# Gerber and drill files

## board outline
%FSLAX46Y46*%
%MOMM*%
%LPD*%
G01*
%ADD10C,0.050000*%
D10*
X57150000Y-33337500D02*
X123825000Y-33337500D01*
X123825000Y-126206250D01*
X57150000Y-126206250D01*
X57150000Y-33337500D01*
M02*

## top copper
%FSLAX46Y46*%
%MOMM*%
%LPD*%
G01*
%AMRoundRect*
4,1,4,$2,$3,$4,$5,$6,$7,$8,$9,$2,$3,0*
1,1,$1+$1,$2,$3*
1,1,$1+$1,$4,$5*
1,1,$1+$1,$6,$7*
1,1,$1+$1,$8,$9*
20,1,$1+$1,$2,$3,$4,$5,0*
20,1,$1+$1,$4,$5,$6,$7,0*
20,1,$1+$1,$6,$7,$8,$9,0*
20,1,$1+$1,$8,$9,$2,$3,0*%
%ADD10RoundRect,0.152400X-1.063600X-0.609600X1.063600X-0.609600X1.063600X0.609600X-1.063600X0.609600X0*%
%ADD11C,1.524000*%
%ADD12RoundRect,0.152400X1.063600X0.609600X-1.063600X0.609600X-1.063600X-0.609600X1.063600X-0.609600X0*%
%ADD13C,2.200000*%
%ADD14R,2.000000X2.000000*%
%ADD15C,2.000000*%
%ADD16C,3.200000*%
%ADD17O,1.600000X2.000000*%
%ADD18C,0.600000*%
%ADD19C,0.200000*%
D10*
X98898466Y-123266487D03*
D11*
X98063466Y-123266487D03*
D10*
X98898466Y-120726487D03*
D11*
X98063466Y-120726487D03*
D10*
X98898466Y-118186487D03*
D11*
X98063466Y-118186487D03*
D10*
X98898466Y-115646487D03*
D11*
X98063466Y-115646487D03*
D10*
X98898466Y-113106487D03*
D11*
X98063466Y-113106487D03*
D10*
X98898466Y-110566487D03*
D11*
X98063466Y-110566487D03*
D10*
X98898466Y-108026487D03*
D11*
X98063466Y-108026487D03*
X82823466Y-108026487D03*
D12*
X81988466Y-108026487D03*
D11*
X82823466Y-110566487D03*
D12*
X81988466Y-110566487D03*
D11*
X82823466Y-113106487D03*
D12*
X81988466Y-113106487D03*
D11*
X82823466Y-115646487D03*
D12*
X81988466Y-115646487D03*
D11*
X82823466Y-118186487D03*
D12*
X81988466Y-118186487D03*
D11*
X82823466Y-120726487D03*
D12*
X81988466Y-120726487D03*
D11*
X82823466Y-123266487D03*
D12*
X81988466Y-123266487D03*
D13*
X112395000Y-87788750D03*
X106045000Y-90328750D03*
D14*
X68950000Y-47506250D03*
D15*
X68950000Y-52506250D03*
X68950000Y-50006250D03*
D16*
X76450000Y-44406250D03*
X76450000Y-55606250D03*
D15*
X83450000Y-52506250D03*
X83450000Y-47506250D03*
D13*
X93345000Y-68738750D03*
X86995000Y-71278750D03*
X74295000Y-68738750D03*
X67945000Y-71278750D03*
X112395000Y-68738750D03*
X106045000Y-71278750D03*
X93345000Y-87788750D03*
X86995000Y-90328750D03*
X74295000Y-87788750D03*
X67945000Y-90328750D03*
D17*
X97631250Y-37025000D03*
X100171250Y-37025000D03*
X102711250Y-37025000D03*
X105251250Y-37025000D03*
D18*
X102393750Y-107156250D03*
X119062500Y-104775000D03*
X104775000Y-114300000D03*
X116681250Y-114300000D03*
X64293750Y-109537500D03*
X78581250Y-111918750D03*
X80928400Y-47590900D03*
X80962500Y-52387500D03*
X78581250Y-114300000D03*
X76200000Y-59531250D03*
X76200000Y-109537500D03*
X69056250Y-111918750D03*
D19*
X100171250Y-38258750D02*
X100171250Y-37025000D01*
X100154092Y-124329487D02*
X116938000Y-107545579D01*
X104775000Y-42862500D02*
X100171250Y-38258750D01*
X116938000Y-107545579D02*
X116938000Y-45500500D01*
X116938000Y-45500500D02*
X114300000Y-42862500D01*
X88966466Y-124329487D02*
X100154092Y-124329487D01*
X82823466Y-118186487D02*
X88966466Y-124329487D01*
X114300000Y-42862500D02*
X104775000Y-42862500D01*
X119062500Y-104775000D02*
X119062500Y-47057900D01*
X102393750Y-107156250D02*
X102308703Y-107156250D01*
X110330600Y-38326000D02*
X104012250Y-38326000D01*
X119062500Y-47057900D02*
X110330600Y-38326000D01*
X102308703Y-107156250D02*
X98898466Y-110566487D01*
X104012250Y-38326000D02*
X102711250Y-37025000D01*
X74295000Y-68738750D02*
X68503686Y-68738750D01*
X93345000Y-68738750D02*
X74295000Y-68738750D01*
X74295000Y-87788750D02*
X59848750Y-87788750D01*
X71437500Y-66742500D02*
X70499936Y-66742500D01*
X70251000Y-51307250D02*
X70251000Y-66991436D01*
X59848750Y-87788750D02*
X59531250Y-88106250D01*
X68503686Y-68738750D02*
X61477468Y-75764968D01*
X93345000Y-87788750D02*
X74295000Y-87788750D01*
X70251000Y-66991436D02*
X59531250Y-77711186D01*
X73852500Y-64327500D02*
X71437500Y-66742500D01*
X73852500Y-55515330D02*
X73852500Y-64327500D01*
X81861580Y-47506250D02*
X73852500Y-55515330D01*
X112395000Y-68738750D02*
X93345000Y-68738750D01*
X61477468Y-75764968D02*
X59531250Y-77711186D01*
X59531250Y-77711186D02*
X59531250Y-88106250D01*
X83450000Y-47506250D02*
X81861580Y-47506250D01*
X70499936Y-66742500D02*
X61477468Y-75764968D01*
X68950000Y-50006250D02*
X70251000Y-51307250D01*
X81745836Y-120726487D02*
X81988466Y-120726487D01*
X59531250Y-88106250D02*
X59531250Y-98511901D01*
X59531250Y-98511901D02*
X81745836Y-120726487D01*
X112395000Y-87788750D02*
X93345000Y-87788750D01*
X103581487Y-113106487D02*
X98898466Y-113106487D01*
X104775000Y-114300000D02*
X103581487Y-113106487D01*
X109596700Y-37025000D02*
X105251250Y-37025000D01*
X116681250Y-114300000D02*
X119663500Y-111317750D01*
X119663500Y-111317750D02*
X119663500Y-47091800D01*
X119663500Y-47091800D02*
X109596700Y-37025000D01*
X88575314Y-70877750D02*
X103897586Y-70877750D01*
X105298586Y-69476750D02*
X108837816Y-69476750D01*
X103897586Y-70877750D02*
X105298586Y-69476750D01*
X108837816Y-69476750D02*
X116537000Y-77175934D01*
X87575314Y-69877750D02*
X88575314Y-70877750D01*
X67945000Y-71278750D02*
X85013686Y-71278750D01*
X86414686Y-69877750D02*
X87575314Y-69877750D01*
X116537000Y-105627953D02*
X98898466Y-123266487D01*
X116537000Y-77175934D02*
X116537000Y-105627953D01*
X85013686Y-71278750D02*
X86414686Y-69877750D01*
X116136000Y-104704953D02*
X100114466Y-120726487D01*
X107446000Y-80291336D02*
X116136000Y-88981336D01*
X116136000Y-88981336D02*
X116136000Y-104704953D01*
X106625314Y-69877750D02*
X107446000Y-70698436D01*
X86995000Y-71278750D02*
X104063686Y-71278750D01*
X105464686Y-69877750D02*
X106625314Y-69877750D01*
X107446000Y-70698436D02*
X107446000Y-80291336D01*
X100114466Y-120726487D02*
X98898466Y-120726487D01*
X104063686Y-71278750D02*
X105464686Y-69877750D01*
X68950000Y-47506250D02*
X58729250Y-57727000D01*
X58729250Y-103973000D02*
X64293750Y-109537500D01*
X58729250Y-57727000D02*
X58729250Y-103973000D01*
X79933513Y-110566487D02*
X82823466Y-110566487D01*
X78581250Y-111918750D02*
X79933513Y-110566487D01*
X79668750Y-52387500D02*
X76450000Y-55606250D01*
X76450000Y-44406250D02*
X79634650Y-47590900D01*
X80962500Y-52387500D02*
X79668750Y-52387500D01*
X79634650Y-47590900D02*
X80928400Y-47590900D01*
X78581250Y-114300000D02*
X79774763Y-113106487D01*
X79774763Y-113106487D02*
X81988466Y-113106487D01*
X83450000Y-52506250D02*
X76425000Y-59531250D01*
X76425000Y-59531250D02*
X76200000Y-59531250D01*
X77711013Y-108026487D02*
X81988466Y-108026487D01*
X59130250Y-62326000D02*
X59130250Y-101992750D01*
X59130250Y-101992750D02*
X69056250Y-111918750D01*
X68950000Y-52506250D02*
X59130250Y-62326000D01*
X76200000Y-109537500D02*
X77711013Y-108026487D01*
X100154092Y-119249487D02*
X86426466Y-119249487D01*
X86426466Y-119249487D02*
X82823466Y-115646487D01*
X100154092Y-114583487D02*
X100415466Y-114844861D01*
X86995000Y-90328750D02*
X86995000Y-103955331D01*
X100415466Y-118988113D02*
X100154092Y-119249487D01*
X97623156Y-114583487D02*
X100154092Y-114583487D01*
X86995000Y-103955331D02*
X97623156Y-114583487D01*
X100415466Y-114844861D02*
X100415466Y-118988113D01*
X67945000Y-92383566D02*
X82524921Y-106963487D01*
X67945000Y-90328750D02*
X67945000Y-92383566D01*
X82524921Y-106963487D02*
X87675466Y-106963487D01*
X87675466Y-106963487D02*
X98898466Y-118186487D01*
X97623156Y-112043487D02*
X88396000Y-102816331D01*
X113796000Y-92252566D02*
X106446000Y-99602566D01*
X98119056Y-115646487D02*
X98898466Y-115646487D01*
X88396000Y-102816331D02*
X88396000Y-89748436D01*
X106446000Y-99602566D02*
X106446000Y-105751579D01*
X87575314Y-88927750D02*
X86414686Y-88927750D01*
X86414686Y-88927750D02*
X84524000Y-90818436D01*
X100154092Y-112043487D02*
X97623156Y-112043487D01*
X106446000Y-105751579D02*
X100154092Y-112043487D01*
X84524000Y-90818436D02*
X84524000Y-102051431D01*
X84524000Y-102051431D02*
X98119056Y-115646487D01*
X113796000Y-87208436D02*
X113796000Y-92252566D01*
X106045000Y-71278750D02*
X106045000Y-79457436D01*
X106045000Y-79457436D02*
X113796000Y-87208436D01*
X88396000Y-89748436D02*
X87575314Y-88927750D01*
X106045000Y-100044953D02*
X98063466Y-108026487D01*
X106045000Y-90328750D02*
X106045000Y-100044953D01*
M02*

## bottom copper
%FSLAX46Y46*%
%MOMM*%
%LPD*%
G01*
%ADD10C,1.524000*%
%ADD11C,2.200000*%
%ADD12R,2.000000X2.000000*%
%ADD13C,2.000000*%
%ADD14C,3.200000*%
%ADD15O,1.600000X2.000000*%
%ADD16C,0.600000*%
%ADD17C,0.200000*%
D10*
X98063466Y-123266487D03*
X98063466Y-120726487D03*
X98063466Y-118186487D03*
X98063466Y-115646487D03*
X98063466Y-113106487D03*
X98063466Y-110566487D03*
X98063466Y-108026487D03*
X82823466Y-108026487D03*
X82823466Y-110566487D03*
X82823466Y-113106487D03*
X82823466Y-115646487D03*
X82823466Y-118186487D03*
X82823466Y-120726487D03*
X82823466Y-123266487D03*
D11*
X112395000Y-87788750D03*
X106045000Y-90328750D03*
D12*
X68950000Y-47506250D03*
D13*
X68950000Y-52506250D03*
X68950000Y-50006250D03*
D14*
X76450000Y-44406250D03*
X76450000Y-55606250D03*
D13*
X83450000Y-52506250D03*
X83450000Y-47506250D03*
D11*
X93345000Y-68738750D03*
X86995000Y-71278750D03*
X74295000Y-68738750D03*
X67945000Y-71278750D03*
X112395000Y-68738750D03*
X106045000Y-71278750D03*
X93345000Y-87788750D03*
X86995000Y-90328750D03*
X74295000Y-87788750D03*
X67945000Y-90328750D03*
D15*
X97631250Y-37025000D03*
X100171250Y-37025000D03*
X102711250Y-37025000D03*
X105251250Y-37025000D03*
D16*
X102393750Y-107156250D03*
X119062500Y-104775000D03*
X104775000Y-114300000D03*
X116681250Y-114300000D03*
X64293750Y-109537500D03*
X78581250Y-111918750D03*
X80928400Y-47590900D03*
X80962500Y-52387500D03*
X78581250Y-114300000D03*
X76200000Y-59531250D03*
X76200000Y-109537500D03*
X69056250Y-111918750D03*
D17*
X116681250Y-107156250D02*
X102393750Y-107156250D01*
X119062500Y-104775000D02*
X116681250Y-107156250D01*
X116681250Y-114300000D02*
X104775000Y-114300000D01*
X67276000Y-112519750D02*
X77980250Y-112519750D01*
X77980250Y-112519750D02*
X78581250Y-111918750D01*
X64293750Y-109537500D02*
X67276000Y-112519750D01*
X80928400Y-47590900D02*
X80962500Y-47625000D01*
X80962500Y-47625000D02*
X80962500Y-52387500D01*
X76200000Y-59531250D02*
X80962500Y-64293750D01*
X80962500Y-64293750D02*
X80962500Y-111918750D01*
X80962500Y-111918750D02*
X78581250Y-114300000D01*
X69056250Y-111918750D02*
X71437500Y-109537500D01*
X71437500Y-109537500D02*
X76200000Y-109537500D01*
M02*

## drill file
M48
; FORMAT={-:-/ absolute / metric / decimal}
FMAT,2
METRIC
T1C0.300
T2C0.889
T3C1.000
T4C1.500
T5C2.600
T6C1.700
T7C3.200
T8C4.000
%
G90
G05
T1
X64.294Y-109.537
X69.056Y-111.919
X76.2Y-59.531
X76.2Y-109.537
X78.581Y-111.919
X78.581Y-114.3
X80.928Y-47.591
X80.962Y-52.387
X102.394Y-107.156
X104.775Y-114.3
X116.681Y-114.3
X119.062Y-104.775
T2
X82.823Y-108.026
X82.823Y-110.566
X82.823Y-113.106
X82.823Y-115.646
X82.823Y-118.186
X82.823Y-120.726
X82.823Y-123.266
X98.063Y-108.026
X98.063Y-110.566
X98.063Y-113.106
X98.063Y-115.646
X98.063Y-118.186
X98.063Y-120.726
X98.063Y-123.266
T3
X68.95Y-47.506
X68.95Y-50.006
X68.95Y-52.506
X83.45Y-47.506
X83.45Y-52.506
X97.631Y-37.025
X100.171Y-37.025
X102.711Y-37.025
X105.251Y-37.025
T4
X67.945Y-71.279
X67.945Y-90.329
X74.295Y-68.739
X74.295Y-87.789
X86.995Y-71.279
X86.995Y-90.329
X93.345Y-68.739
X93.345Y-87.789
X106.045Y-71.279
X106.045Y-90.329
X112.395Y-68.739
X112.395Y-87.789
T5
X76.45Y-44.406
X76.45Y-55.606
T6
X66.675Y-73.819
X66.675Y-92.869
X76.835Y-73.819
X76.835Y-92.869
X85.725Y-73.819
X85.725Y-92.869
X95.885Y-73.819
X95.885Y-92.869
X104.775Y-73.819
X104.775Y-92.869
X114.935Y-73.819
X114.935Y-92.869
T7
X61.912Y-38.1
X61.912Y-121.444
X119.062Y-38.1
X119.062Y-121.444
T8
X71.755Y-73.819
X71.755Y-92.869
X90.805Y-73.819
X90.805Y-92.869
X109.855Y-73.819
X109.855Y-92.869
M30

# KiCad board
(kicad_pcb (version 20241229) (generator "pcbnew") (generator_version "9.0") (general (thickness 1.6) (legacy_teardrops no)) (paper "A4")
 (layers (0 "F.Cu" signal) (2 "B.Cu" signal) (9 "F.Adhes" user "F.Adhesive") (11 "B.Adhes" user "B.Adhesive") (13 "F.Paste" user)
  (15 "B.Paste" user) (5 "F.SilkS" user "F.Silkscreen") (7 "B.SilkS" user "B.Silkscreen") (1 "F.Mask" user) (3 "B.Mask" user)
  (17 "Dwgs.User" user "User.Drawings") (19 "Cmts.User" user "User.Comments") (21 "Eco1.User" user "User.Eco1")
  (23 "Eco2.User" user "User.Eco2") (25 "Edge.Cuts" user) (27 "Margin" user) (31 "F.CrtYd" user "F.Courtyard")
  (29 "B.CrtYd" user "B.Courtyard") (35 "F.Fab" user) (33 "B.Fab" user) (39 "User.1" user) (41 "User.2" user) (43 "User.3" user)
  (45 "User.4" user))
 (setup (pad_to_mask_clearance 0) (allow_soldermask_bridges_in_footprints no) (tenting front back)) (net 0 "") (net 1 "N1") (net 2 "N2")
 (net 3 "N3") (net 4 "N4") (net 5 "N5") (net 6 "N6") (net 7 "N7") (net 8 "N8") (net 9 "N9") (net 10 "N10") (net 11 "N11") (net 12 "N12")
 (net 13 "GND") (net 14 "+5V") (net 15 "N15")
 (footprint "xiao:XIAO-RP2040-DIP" (layer "F.Cu") (at 90.443466 115.646487 180)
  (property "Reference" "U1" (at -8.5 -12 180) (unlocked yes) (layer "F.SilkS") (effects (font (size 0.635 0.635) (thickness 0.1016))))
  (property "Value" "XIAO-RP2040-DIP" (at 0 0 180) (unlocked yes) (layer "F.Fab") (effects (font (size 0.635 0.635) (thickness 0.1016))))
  (pad "1" smd roundrect (at -8.455 -7.62) (size 2.432 1.524) (layers "F.Cu" "F.Mask") (roundrect_rratio 0.1) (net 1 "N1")
   (thermal_bridge_angle 45))
  (pad "1" thru_hole circle (at -7.62 -7.62) (size 1.524 1.524) (drill 0.889) (layers "*.Cu" "*.Mask") (remove_unused_layers no)
   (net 1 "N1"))
  (pad "2" smd roundrect (at -8.455 -5.08) (size 2.432 1.524) (layers "F.Cu" "F.Mask") (roundrect_rratio 0.1) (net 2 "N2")
   (thermal_bridge_angle 45))
  (pad "2" thru_hole circle (at -7.62 -5.08) (size 1.524 1.524) (drill 0.889) (layers "*.Cu" "*.Mask") (remove_unused_layers no)
   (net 2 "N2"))
  (pad "3" smd roundrect (at -8.455 -2.54) (size 2.432 1.524) (layers "F.Cu" "F.Mask") (roundrect_rratio 0.1) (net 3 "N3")
   (thermal_bridge_angle 45))
  (pad "3" thru_hole circle (at -7.62 -2.54) (size 1.524 1.524) (drill 0.889) (layers "*.Cu" "*.Mask") (remove_unused_layers no)
   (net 3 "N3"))
  (pad "4" smd roundrect (at -8.455 0) (size 2.432 1.524) (layers "F.Cu" "F.Mask") (roundrect_rratio 0.1) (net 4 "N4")
   (thermal_bridge_angle 45))
  (pad "4" thru_hole circle (at -7.62 0) (size 1.524 1.524) (drill 0.889) (layers "*.Cu" "*.Mask") (remove_unused_layers no) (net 4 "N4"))
  (pad "5" smd roundrect (at -8.455 2.54) (size 2.432 1.524) (layers "F.Cu" "F.Mask") (roundrect_rratio 0.1) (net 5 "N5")
   (thermal_bridge_angle 45))
  (pad "5" thru_hole circle (at -7.62 2.54) (size 1.524 1.524) (drill 0.889) (layers "*.Cu" "*.Mask") (remove_unused_layers no) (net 5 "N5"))
  (pad "6" smd roundrect (at -8.455 5.08) (size 2.432 1.524) (layers "F.Cu" "F.Mask") (roundrect_rratio 0.1) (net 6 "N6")
   (thermal_bridge_angle 45))
  (pad "6" thru_hole circle (at -7.62 5.08) (size 1.524 1.524) (drill 0.889) (layers "*.Cu" "*.Mask") (remove_unused_layers no) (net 6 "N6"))
  (pad "7" smd roundrect (at -8.455 7.62) (size 2.432 1.524) (layers "F.Cu" "F.Mask") (roundrect_rratio 0.1) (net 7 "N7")
   (thermal_bridge_angle 45))
  (pad "7" thru_hole circle (at -7.62 7.62) (size 1.524 1.524) (drill 0.889) (layers "*.Cu" "*.Mask") (remove_unused_layers no) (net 7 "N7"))
  (pad "8" thru_hole circle (at 7.62 7.62 180) (size 1.524 1.524) (drill 0.889) (layers "*.Cu" "*.Mask") (remove_unused_layers no)
   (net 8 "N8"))
  (pad "8" smd roundrect (at 8.455 7.62 180) (size 2.432 1.524) (layers "F.Cu" "F.Mask") (roundrect_rratio 0.1) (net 8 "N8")
   (thermal_bridge_angle 45))
  (pad "9" thru_hole circle (at 7.62 5.08 180) (size 1.524 1.524) (drill 0.889) (layers "*.Cu" "*.Mask") (remove_unused_layers no)
   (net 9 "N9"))
  (pad "9" smd roundrect (at 8.455 5.08 180) (size 2.432 1.524) (layers "F.Cu" "F.Mask") (roundrect_rratio 0.1) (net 9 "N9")
   (thermal_bridge_angle 45))
  (pad "10" thru_hole circle (at 7.62 2.54 180) (size 1.524 1.524) (drill 0.889) (layers "*.Cu" "*.Mask") (remove_unused_layers no)
   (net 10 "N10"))
  (pad "10" smd roundrect (at 8.455 2.54 180) (size 2.432 1.524) (layers "F.Cu" "F.Mask") (roundrect_rratio 0.1) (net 10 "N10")
   (thermal_bridge_angle 45))
  (pad "11" thru_hole circle (at 7.62 0 180) (size 1.524 1.524) (drill 0.889) (layers "*.Cu" "*.Mask") (remove_unused_layers no)
   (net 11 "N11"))
  (pad "11" smd roundrect (at 8.455 0 180) (size 2.432 1.524) (layers "F.Cu" "F.Mask") (roundrect_rratio 0.1) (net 11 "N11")
   (thermal_bridge_angle 45))
  (pad "12" thru_hole circle (at 7.62 -2.54 180) (size 1.524 1.524) (drill 0.889) (layers "*.Cu" "*.Mask") (remove_unused_layers no)
   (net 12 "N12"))
  (pad "12" smd roundrect (at 8.455 -2.54 180) (size 2.432 1.524) (layers "F.Cu" "F.Mask") (roundrect_rratio 0.1) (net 12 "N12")
   (thermal_bridge_angle 45))
  (pad "13" thru_hole circle (at 7.62 -5.08 180) (size 1.524 1.524) (drill 0.889) (layers "*.Cu" "*.Mask") (remove_unused_layers no)
   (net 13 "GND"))
  (pad "13" smd roundrect (at 8.455 -5.08 180) (size 2.432 1.524) (layers "F.Cu" "F.Mask") (roundrect_rratio 0.1) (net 13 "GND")
   (thermal_bridge_angle 45))
  (pad "14" thru_hole circle (at 7.62 -7.62 180) (size 1.524 1.524) (drill 0.889) (layers "*.Cu" "*.Mask") (remove_unused_layers no)
   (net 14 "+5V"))
  (pad "14" smd roundrect (at 8.455 -7.62 180) (size 2.432 1.524) (layers "F.Cu" "F.Mask") (roundrect_rratio 0.1) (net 14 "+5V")
   (thermal_bridge_angle 45)))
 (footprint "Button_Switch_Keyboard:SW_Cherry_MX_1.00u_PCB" (layer "F.Cu") (at 112.395 87.78875)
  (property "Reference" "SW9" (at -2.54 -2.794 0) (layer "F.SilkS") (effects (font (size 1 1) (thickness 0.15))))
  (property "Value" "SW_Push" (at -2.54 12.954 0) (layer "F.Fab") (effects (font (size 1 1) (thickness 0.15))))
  (pad "" np_thru_hole circle (at -7.62 5.08) (size 1.7 1.7) (drill 1.7) (layers "*.Cu" "*.Mask"))
  (pad "" np_thru_hole circle (at -2.54 5.08) (size 4 4) (drill 4) (layers "*.Cu" "*.Mask"))
  (pad "" np_thru_hole circle (at 2.54 5.08) (size 1.7 1.7) (drill 1.7) (layers "*.Cu" "*.Mask"))
  (pad "1" thru_hole circle (at 0 0) (size 2.2 2.2) (drill 1.5) (layers "*.Cu" "*.Mask") (remove_unused_layers no) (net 13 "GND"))
  (pad "2" thru_hole circle (at -6.35 2.54) (size 2.2 2.2) (drill 1.5) (layers "*.Cu" "*.Mask") (remove_unused_layers no) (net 7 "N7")))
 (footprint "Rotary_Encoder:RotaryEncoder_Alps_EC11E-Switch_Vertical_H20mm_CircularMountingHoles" (layer "F.Cu") (at 68.95 47.50625)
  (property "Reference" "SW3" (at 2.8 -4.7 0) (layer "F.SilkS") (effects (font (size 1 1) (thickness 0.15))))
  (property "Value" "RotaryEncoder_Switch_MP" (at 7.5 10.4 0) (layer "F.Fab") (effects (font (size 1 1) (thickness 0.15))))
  (pad "A" thru_hole rect (at 0 0) (size 2 2) (drill 1) (layers "*.Cu" "*.Mask") (remove_unused_layers no) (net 9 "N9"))
  (pad "B" thru_hole circle (at 0 5) (size 2 2) (drill 1) (layers "*.Cu" "*.Mask") (remove_unused_layers no) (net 8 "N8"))
  (pad "C" thru_hole circle (at 0 2.5) (size 2 2) (drill 1) (layers "*.Cu" "*.Mask") (remove_unused_layers no) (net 13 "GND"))
  (pad "MP" thru_hole circle (at 7.5 -3.1) (size 3.2 3.2) (drill 2.6) (layers "*.Cu" "*.Mask") (remove_unused_layers no) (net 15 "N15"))
  (pad "MP" thru_hole circle (at 7.5 8.1) (size 3.2 3.2) (drill 2.6) (layers "*.Cu" "*.Mask") (remove_unused_layers no) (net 15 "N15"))
  (pad "S1" thru_hole circle (at 14.5 5) (size 2 2) (drill 1) (layers "*.Cu" "*.Mask") (remove_unused_layers no) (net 10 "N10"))
  (pad "S2" thru_hole circle (at 14.5 0) (size 2 2) (drill 1) (layers "*.Cu" "*.Mask") (remove_unused_layers no) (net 13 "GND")))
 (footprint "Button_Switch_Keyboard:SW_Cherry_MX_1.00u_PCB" (layer "F.Cu") (at 93.345 68.73875)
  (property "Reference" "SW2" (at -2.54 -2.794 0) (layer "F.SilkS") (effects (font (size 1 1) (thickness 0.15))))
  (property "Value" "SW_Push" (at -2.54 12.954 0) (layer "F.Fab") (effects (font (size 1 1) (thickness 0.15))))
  (pad "" np_thru_hole circle (at -7.62 5.08) (size 1.7 1.7) (drill 1.7) (layers "*.Cu" "*.Mask"))
  (pad "" np_thru_hole circle (at -2.54 5.08) (size 4 4) (drill 4) (layers "*.Cu" "*.Mask"))
  (pad "" np_thru_hole circle (at 2.54 5.08) (size 1.7 1.7) (drill 1.7) (layers "*.Cu" "*.Mask"))
  (pad "1" thru_hole circle (at 0 0) (size 2.2 2.2) (drill 1.5) (layers "*.Cu" "*.Mask") (remove_unused_layers no) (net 13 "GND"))
  (pad "2" thru_hole circle (at -6.35 2.54) (size 2.2 2.2) (drill 1.5) (layers "*.Cu" "*.Mask") (remove_unused_layers no) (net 2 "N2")))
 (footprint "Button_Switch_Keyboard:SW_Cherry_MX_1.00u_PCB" (layer "F.Cu") (at 74.295 68.73875)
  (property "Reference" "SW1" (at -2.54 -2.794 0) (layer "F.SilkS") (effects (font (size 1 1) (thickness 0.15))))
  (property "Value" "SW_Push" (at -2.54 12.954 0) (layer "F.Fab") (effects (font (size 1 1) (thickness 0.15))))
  (pad "" np_thru_hole circle (at -7.62 5.08) (size 1.7 1.7) (drill 1.7) (layers "*.Cu" "*.Mask"))
  (pad "" np_thru_hole circle (at -2.54 5.08) (size 4 4) (drill 4) (layers "*.Cu" "*.Mask"))
  (pad "" np_thru_hole circle (at 2.54 5.08) (size 1.7 1.7) (drill 1.7) (layers "*.Cu" "*.Mask"))
  (pad "1" thru_hole circle (at 0 0) (size 2.2 2.2) (drill 1.5) (layers "*.Cu" "*.Mask") (remove_unused_layers no) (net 13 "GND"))
  (pad "2" thru_hole circle (at -6.35 2.54) (size 2.2 2.2) (drill 1.5) (layers "*.Cu" "*.Mask") (remove_unused_layers no) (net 1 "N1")))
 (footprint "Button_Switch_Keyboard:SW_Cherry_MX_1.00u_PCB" (layer "F.Cu") (at 112.395 68.73875)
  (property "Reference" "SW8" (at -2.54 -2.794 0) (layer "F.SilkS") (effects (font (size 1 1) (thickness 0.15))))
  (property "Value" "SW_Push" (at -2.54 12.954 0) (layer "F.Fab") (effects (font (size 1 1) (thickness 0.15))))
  (pad "" np_thru_hole circle (at -7.62 5.08) (size 1.7 1.7) (drill 1.7) (layers "*.Cu" "*.Mask"))
  (pad "" np_thru_hole circle (at -2.54 5.08) (size 4 4) (drill 4) (layers "*.Cu" "*.Mask"))
  (pad "" np_thru_hole circle (at 2.54 5.08) (size 1.7 1.7) (drill 1.7) (layers "*.Cu" "*.Mask"))
  (pad "1" thru_hole circle (at 0 0) (size 2.2 2.2) (drill 1.5) (layers "*.Cu" "*.Mask") (remove_unused_layers no) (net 13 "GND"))
  (pad "2" thru_hole circle (at -6.35 2.54) (size 2.2 2.2) (drill 1.5) (layers "*.Cu" "*.Mask") (remove_unused_layers no) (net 4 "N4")))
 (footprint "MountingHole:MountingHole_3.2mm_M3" (layer "F.Cu") (at 119.0625 38.1)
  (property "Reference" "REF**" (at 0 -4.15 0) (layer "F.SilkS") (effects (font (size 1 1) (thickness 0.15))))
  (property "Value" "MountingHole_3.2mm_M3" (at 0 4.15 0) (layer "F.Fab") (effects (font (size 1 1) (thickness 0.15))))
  (pad "" np_thru_hole circle (at 0 0) (size 3.2 3.2) (drill 3.2) (layers "*.Cu" "*.Mask")))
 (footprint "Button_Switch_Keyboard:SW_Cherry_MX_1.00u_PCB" (layer "F.Cu") (at 93.345 87.78875)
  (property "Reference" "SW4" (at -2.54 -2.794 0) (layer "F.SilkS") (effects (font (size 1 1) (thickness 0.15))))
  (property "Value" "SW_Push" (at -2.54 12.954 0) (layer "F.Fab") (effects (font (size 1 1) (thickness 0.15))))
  (pad "" np_thru_hole circle (at -7.62 5.08) (size 1.7 1.7) (drill 1.7) (layers "*.Cu" "*.Mask"))
  (pad "" np_thru_hole circle (at -2.54 5.08) (size 4 4) (drill 4) (layers "*.Cu" "*.Mask"))
  (pad "" np_thru_hole circle (at 2.54 5.08) (size 1.7 1.7) (drill 1.7) (layers "*.Cu" "*.Mask"))
  (pad "1" thru_hole circle (at 0 0) (size 2.2 2.2) (drill 1.5) (layers "*.Cu" "*.Mask") (remove_unused_layers no) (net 13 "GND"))
  (pad "2" thru_hole circle (at -6.35 2.54) (size 2.2 2.2) (drill 1.5) (layers "*.Cu" "*.Mask") (remove_unused_layers no) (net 11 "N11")))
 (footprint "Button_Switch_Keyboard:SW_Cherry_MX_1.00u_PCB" (layer "F.Cu") (at 74.295 87.78875)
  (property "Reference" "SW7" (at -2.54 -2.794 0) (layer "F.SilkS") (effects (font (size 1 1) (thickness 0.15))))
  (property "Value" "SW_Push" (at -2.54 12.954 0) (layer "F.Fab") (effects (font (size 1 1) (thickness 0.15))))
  (pad "" np_thru_hole circle (at -7.62 5.08) (size 1.7 1.7) (drill 1.7) (layers "*.Cu" "*.Mask"))
  (pad "" np_thru_hole circle (at -2.54 5.08) (size 4 4) (drill 4) (layers "*.Cu" "*.Mask"))
  (pad "" np_thru_hole circle (at 2.54 5.08) (size 1.7 1.7) (drill 1.7) (layers "*.Cu" "*.Mask"))
  (pad "1" thru_hole circle (at 0 0) (size 2.2 2.2) (drill 1.5) (layers "*.Cu" "*.Mask") (remove_unused_layers no) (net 13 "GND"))
  (pad "2" thru_hole circle (at -6.35 2.54) (size 2.2 2.2) (drill 1.5) (layers "*.Cu" "*.Mask") (remove_unused_layers no) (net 3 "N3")))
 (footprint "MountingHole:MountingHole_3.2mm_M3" (layer "F.Cu") (at 119.0625 121.44375)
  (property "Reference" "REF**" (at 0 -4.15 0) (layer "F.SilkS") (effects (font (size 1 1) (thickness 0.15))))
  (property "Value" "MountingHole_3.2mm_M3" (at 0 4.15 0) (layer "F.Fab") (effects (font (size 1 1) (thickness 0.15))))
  (pad "" np_thru_hole circle (at 0 0) (size 3.2 3.2) (drill 3.2) (layers "*.Cu" "*.Mask")))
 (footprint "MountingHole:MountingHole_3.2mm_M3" (layer "F.Cu") (at 61.9125 38.1)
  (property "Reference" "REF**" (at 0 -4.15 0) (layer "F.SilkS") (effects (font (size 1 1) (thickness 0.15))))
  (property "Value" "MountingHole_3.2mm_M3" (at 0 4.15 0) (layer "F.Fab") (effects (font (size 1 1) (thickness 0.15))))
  (pad "" np_thru_hole circle (at 0 0) (size 3.2 3.2) (drill 3.2) (layers "*.Cu" "*.Mask")))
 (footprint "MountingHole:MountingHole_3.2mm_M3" (layer "F.Cu") (at 61.9125 121.44375)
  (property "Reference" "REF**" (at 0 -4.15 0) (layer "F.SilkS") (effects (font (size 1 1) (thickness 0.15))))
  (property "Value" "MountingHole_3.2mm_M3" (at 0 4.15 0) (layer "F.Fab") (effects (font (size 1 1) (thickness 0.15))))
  (pad "" np_thru_hole circle (at 0 0) (size 3.2 3.2) (drill 3.2) (layers "*.Cu" "*.Mask")))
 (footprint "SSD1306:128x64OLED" (layer "F.Cu") (at 101.25125 47.625)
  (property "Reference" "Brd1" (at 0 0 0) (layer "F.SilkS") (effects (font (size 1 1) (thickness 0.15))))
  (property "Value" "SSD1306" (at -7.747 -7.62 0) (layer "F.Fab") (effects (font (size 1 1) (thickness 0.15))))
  (pad "1" thru_hole oval (at -3.62 -10.6 90) (size 2 1.6) (drill 1) (layers "*.Cu" "*.Mask") (remove_unused_layers no) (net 13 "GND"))
  (pad "2" thru_hole oval (at -1.08 -10.6 90) (size 2 1.6) (drill 1) (layers "*.Cu" "*.Mask") (remove_unused_layers no) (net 12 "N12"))
  (pad "3" thru_hole oval (at 1.46 -10.6 90) (size 2 1.6) (drill 1) (layers "*.Cu" "*.Mask") (remove_unused_layers no) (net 6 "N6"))
  (pad "4" thru_hole oval (at 4 -10.6 90) (size 2 1.6) (drill 1) (layers "*.Cu" "*.Mask") (remove_unused_layers no) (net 5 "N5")))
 (gr_rect (start 57.15 33.3375) (end 123.825 126.20625) (stroke (width 0.05) (type default)) (fill no) (layer "Edge.Cuts"))
 (segment (start 100.17125 38.25875) (end 100.17125 37.025) (width 0.2) (layer "F.Cu") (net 12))
 (segment (start 100.154092 124.329487) (end 116.938 107.545579) (width 0.2) (layer "F.Cu") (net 12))
 (segment (start 104.775 42.8625) (end 100.17125 38.25875) (width 0.2) (layer "F.Cu") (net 12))
 (segment (start 116.938 107.545579) (end 116.938 45.5005) (width 0.2) (layer "F.Cu") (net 12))
 (segment (start 116.938 45.5005) (end 114.3 42.8625) (width 0.2) (layer "F.Cu") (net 12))
 (segment (start 88.966466 124.329487) (end 100.154092 124.329487) (width 0.2) (layer "F.Cu") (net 12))
 (segment (start 82.823466 118.186487) (end 88.966466 124.329487) (width 0.2) (layer "F.Cu") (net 12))
 (segment (start 114.3 42.8625) (end 104.775 42.8625) (width 0.2) (layer "F.Cu") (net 12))
 (segment (start 119.0625 104.775) (end 119.0625 47.0579) (width 0.2) (layer "F.Cu") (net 6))
 (segment (start 102.39375 107.15625) (end 102.308703 107.15625) (width 0.2) (layer "F.Cu") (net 6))
 (segment (start 110.3306 38.326) (end 104.01225 38.326) (width 0.2) (layer "F.Cu") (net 6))
 (segment (start 119.0625 47.0579) (end 110.3306 38.326) (width 0.2) (layer "F.Cu") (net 6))
 (segment (start 102.308703 107.15625) (end 98.898466 110.566487) (width 0.2) (layer "F.Cu") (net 6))
 (segment (start 104.01225 38.326) (end 102.71125 37.025) (width 0.2) (layer "F.Cu") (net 6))
 (via (at 102.39375 107.15625) (size 0.6) (drill 0.3) (layers "F.Cu" "B.Cu") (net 6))
 (via (at 119.0625 104.775) (size 0.6) (drill 0.3) (layers "F.Cu" "B.Cu") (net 6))
 (segment (start 116.68125 107.15625) (end 102.39375 107.15625) (width 0.2) (layer "B.Cu") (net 6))
 (segment (start 119.0625 104.775) (end 116.68125 107.15625) (width 0.2) (layer "B.Cu") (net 6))
 (segment (start 74.295 68.73875) (end 68.503686 68.73875) (width 0.2) (layer "F.Cu") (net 13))
 (segment (start 93.345 68.73875) (end 74.295 68.73875) (width 0.2) (layer "F.Cu") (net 13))
 (segment (start 74.295 87.78875) (end 59.84875 87.78875) (width 0.2) (layer "F.Cu") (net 13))
 (segment (start 71.4375 66.7425) (end 70.499936 66.7425) (width 0.2) (layer "F.Cu") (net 13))
 (segment (start 70.251 51.30725) (end 70.251 66.991436) (width 0.2) (layer "F.Cu") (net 13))
 (segment (start 59.84875 87.78875) (end 59.53125 88.10625) (width 0.2) (layer "F.Cu") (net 13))
 (segment (start 68.503686 68.73875) (end 61.477468 75.764968) (width 0.2) (layer "F.Cu") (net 13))
 (segment (start 93.345 87.78875) (end 74.295 87.78875) (width 0.2) (layer "F.Cu") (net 13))
 (segment (start 70.251 66.991436) (end 59.53125 77.711186) (width 0.2) (layer "F.Cu") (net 13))
 (segment (start 73.8525 64.3275) (end 71.4375 66.7425) (width 0.2) (layer "F.Cu") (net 13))
 (segment (start 73.8525 55.51533) (end 73.8525 64.3275) (width 0.2) (layer "F.Cu") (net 13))
 (segment (start 81.86158 47.50625) (end 73.8525 55.51533) (width 0.2) (layer "F.Cu") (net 13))
 (segment (start 112.395 68.73875) (end 93.345 68.73875) (width 0.2) (layer "F.Cu") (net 13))
 (segment (start 61.477468 75.764968) (end 59.53125 77.711186) (width 0.2) (layer "F.Cu") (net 13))
 (segment (start 59.53125 77.711186) (end 59.53125 88.10625) (width 0.2) (layer "F.Cu") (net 13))
 (segment (start 83.45 47.50625) (end 81.86158 47.50625) (width 0.2) (layer "F.Cu") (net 13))
 (segment (start 70.499936 66.7425) (end 61.477468 75.764968) (width 0.2) (layer "F.Cu") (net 13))
 (segment (start 68.95 50.00625) (end 70.251 51.30725) (width 0.2) (layer "F.Cu") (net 13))
 (segment (start 81.745836 120.726487) (end 81.988466 120.726487) (width 0.2) (layer "F.Cu") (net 13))
 (segment (start 59.53125 88.10625) (end 59.53125 98.511901) (width 0.2) (layer "F.Cu") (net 13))
 (segment (start 59.53125 98.511901) (end 81.745836 120.726487) (width 0.2) (layer "F.Cu") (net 13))
 (segment (start 112.395 87.78875) (end 93.345 87.78875) (width 0.2) (layer "F.Cu") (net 13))
 (segment (start 103.581487 113.106487) (end 98.898466 113.106487) (width 0.2) (layer "F.Cu") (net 5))
 (segment (start 104.775 114.3) (end 103.581487 113.106487) (width 0.2) (layer "F.Cu") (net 5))
 (segment (start 109.5967 37.025) (end 105.25125 37.025) (width 0.2) (layer "F.Cu") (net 5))
 (segment (start 116.68125 114.3) (end 119.6635 111.31775) (width 0.2) (layer "F.Cu") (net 5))
 (segment (start 119.6635 111.31775) (end 119.6635 47.0918) (width 0.2) (layer "F.Cu") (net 5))
 (segment (start 119.6635 47.0918) (end 109.5967 37.025) (width 0.2) (layer "F.Cu") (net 5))
 (via (at 104.775 114.3) (size 0.6) (drill 0.3) (layers "F.Cu" "B.Cu") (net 5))
 (via (at 116.68125 114.3) (size 0.6) (drill 0.3) (layers "F.Cu" "B.Cu") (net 5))
 (segment (start 116.68125 114.3) (end 104.775 114.3) (width 0.2) (layer "B.Cu") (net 5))
 (segment (start 88.575314 70.87775) (end 103.897586 70.87775) (width 0.2) (layer "F.Cu") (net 1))
 (segment (start 105.298586 69.47675) (end 108.837816 69.47675) (width 0.2) (layer "F.Cu") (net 1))
 (segment (start 103.897586 70.87775) (end 105.298586 69.47675) (width 0.2) (layer "F.Cu") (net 1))
 (segment (start 108.837816 69.47675) (end 116.537 77.175934) (width 0.2) (layer "F.Cu") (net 1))
 (segment (start 87.575314 69.87775) (end 88.575314 70.87775) (width 0.2) (layer "F.Cu") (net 1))
 (segment (start 67.945 71.27875) (end 85.013686 71.27875) (width 0.2) (layer "F.Cu") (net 1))
 (segment (start 86.414686 69.87775) (end 87.575314 69.87775) (width 0.2) (layer "F.Cu") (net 1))
 (segment (start 116.537 105.627953) (end 98.898466 123.266487) (width 0.2) (layer "F.Cu") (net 1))
 (segment (start 116.537 77.175934) (end 116.537 105.627953) (width 0.2) (layer "F.Cu") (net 1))
 (segment (start 85.013686 71.27875) (end 86.414686 69.87775) (width 0.2) (layer "F.Cu") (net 1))
 (segment (start 116.136 104.704953) (end 100.114466 120.726487) (width 0.2) (layer "F.Cu") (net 2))
 (segment (start 107.446 80.291336) (end 116.136 88.981336) (width 0.2) (layer "F.Cu") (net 2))
 (segment (start 116.136 88.981336) (end 116.136 104.704953) (width 0.2) (layer "F.Cu") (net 2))
 (segment (start 106.625314 69.87775) (end 107.446 70.698436) (width 0.2) (layer "F.Cu") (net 2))
 (segment (start 86.995 71.27875) (end 104.063686 71.27875) (width 0.2) (layer "F.Cu") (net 2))
 (segment (start 105.464686 69.87775) (end 106.625314 69.87775) (width 0.2) (layer "F.Cu") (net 2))
 (segment (start 107.446 70.698436) (end 107.446 80.291336) (width 0.2) (layer "F.Cu") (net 2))
 (segment (start 100.114466 120.726487) (end 98.898466 120.726487) (width 0.2) (layer "F.Cu") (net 2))
 (segment (start 104.063686 71.27875) (end 105.464686 69.87775) (width 0.2) (layer "F.Cu") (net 2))
 (segment (start 68.95 47.50625) (end 58.72925 57.727) (width 0.2) (layer "F.Cu") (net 9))
 (segment (start 58.72925 103.973) (end 64.29375 109.5375) (width 0.2) (layer "F.Cu") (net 9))
 (segment (start 58.72925 57.727) (end 58.72925 103.973) (width 0.2) (layer "F.Cu") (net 9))
 (segment (start 79.933513 110.566487) (end 82.823466 110.566487) (width 0.2) (layer "F.Cu") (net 9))
 (segment (start 78.58125 111.91875) (end 79.933513 110.566487) (width 0.2) (layer "F.Cu") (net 9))
 (via (at 64.29375 109.5375) (size 0.6) (drill 0.3) (layers "F.Cu" "B.Cu") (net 9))
 (via (at 78.58125 111.91875) (size 0.6) (drill 0.3) (layers "F.Cu" "B.Cu") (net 9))
 (segment (start 67.276 112.51975) (end 77.98025 112.51975) (width 0.2) (layer "B.Cu") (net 9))
 (segment (start 77.98025 112.51975) (end 78.58125 111.91875) (width 0.2) (layer "B.Cu") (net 9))
 (segment (start 64.29375 109.5375) (end 67.276 112.51975) (width 0.2) (layer "B.Cu") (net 9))
 (segment (start 79.66875 52.3875) (end 76.45 55.60625) (width 0.2) (layer "F.Cu") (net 15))
 (segment (start 76.45 44.40625) (end 79.63465 47.5909) (width 0.2) (layer "F.Cu") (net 15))
 (segment (start 80.9625 52.3875) (end 79.66875 52.3875) (width 0.2) (layer "F.Cu") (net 15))
 (segment (start 79.63465 47.5909) (end 80.9284 47.5909) (width 0.2) (layer "F.Cu") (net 15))
 (via (at 80.9284 47.5909) (size 0.6) (drill 0.3) (layers "F.Cu" "B.Cu") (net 15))
 (via (at 80.9625 52.3875) (size 0.6) (drill 0.3) (layers "F.Cu" "B.Cu") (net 15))
 (segment (start 80.9284 47.5909) (end 80.9625 47.625) (width 0.2) (layer "B.Cu") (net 15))
 (segment (start 80.9625 47.625) (end 80.9625 52.3875) (width 0.2) (layer "B.Cu") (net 15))
 (segment (start 78.58125 114.3) (end 79.774763 113.106487) (width 0.2) (layer "F.Cu") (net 10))
 (segment (start 79.774763 113.106487) (end 81.988466 113.106487) (width 0.2) (layer "F.Cu") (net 10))
 (segment (start 83.45 52.50625) (end 76.425 59.53125) (width 0.2) (layer "F.Cu") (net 10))
 (segment (start 76.425 59.53125) (end 76.2 59.53125) (width 0.2) (layer "F.Cu") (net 10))
 (via (at 78.58125 114.3) (size 0.6) (drill 0.3) (layers "F.Cu" "B.Cu") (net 10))
 (via (at 76.2 59.53125) (size 0.6) (drill 0.3) (layers "F.Cu" "B.Cu") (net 10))
 (segment (start 76.2 59.53125) (end 80.9625 64.29375) (width 0.2) (layer "B.Cu") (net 10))
 (segment (start 80.9625 64.29375) (end 80.9625 111.91875) (width 0.2) (layer "B.Cu") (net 10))
 (segment (start 80.9625 111.91875) (end 78.58125 114.3) (width 0.2) (layer "B.Cu") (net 10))
 (segment (start 77.711013 108.026487) (end 81.988466 108.026487) (width 0.2) (layer "F.Cu") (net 8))
 (segment (start 59.13025 62.326) (end 59.13025 101.99275) (width 0.2) (layer "F.Cu") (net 8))
 (segment (start 59.13025 101.99275) (end 69.05625 111.91875) (width 0.2) (layer "F.Cu") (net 8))
 (segment (start 68.95 52.50625) (end 59.13025 62.326) (width 0.2) (layer "F.Cu") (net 8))
 (segment (start 76.2 109.5375) (end 77.711013 108.026487) (width 0.2) (layer "F.Cu") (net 8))
 (via (at 76.2 109.5375) (size 0.6) (drill 0.3) (layers "F.Cu" "B.Cu") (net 8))
 (via (at 69.05625 111.91875) (size 0.6) (drill 0.3) (layers "F.Cu" "B.Cu") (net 8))
 (segment (start 69.05625 111.91875) (end 71.4375 109.5375) (width 0.2) (layer "B.Cu") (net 8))
 (segment (start 71.4375 109.5375) (end 76.2 109.5375) (width 0.2) (layer "B.Cu") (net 8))
 (segment (start 100.154092 119.249487) (end 86.426466 119.249487) (width 0.2) (layer "F.Cu") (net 11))
 (segment (start 86.426466 119.249487) (end 82.823466 115.646487) (width 0.2) (layer "F.Cu") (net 11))
 (segment (start 100.154092 114.583487) (end 100.415466 114.844861) (width 0.2) (layer "F.Cu") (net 11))
 (segment (start 86.995 90.32875) (end 86.995 103.955331) (width 0.2) (layer "F.Cu") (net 11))
 (segment (start 100.415466 118.988113) (end 100.154092 119.249487) (width 0.2) (layer "F.Cu") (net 11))
 (segment (start 97.623156 114.583487) (end 100.154092 114.583487) (width 0.2) (layer "F.Cu") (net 11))
 (segment (start 86.995 103.955331) (end 97.623156 114.583487) (width 0.2) (layer "F.Cu") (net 11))
 (segment (start 100.415466 114.844861) (end 100.415466 118.988113) (width 0.2) (layer "F.Cu") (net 11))
 (segment (start 67.945 92.383566) (end 82.524921 106.963487) (width 0.2) (layer "F.Cu") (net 3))
 (segment (start 67.945 90.32875) (end 67.945 92.383566) (width 0.2) (layer "F.Cu") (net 3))
 (segment (start 82.524921 106.963487) (end 87.675466 106.963487) (width 0.2) (layer "F.Cu") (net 3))
 (segment (start 87.675466 106.963487) (end 98.898466 118.186487) (width 0.2) (layer "F.Cu") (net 3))
 (segment (start 97.623156 112.043487) (end 88.396 102.816331) (width 0.2) (layer "F.Cu") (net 4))
 (segment (start 113.796 92.252566) (end 106.446 99.602566) (width 0.2) (layer "F.Cu") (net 4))
 (segment (start 98.119056 115.646487) (end 98.898466 115.646487) (width 0.2) (layer "F.Cu") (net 4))
 (segment (start 88.396 102.816331) (end 88.396 89.748436) (width 0.2) (layer "F.Cu") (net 4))
 (segment (start 106.446 99.602566) (end 106.446 105.751579) (width 0.2) (layer "F.Cu") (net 4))
 (segment (start 87.575314 88.92775) (end 86.414686 88.92775) (width 0.2) (layer "F.Cu") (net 4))
 (segment (start 86.414686 88.92775) (end 84.524 90.818436) (width 0.2) (layer "F.Cu") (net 4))
 (segment (start 100.154092 112.043487) (end 97.623156 112.043487) (width 0.2) (layer "F.Cu") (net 4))
 (segment (start 106.446 105.751579) (end 100.154092 112.043487) (width 0.2) (layer "F.Cu") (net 4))
 (segment (start 84.524 90.818436) (end 84.524 102.051431) (width 0.2) (layer "F.Cu") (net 4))
 (segment (start 84.524 102.051431) (end 98.119056 115.646487) (width 0.2) (layer "F.Cu") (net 4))
 (segment (start 113.796 87.208436) (end 113.796 92.252566) (width 0.2) (layer "F.Cu") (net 4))
 (segment (start 106.045 71.27875) (end 106.045 79.457436) (width 0.2) (layer "F.Cu") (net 4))
 (segment (start 106.045 79.457436) (end 113.796 87.208436) (width 0.2) (layer "F.Cu") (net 4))
 (segment (start 88.396 89.748436) (end 87.575314 88.92775) (width 0.2) (layer "F.Cu") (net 4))
 (segment (start 106.045 100.044953) (end 98.063466 108.026487) (width 0.2) (layer "F.Cu") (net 7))
 (segment (start 106.045 90.32875) (end 106.045 100.044953) (width 0.2) (layer "F.Cu") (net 7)))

